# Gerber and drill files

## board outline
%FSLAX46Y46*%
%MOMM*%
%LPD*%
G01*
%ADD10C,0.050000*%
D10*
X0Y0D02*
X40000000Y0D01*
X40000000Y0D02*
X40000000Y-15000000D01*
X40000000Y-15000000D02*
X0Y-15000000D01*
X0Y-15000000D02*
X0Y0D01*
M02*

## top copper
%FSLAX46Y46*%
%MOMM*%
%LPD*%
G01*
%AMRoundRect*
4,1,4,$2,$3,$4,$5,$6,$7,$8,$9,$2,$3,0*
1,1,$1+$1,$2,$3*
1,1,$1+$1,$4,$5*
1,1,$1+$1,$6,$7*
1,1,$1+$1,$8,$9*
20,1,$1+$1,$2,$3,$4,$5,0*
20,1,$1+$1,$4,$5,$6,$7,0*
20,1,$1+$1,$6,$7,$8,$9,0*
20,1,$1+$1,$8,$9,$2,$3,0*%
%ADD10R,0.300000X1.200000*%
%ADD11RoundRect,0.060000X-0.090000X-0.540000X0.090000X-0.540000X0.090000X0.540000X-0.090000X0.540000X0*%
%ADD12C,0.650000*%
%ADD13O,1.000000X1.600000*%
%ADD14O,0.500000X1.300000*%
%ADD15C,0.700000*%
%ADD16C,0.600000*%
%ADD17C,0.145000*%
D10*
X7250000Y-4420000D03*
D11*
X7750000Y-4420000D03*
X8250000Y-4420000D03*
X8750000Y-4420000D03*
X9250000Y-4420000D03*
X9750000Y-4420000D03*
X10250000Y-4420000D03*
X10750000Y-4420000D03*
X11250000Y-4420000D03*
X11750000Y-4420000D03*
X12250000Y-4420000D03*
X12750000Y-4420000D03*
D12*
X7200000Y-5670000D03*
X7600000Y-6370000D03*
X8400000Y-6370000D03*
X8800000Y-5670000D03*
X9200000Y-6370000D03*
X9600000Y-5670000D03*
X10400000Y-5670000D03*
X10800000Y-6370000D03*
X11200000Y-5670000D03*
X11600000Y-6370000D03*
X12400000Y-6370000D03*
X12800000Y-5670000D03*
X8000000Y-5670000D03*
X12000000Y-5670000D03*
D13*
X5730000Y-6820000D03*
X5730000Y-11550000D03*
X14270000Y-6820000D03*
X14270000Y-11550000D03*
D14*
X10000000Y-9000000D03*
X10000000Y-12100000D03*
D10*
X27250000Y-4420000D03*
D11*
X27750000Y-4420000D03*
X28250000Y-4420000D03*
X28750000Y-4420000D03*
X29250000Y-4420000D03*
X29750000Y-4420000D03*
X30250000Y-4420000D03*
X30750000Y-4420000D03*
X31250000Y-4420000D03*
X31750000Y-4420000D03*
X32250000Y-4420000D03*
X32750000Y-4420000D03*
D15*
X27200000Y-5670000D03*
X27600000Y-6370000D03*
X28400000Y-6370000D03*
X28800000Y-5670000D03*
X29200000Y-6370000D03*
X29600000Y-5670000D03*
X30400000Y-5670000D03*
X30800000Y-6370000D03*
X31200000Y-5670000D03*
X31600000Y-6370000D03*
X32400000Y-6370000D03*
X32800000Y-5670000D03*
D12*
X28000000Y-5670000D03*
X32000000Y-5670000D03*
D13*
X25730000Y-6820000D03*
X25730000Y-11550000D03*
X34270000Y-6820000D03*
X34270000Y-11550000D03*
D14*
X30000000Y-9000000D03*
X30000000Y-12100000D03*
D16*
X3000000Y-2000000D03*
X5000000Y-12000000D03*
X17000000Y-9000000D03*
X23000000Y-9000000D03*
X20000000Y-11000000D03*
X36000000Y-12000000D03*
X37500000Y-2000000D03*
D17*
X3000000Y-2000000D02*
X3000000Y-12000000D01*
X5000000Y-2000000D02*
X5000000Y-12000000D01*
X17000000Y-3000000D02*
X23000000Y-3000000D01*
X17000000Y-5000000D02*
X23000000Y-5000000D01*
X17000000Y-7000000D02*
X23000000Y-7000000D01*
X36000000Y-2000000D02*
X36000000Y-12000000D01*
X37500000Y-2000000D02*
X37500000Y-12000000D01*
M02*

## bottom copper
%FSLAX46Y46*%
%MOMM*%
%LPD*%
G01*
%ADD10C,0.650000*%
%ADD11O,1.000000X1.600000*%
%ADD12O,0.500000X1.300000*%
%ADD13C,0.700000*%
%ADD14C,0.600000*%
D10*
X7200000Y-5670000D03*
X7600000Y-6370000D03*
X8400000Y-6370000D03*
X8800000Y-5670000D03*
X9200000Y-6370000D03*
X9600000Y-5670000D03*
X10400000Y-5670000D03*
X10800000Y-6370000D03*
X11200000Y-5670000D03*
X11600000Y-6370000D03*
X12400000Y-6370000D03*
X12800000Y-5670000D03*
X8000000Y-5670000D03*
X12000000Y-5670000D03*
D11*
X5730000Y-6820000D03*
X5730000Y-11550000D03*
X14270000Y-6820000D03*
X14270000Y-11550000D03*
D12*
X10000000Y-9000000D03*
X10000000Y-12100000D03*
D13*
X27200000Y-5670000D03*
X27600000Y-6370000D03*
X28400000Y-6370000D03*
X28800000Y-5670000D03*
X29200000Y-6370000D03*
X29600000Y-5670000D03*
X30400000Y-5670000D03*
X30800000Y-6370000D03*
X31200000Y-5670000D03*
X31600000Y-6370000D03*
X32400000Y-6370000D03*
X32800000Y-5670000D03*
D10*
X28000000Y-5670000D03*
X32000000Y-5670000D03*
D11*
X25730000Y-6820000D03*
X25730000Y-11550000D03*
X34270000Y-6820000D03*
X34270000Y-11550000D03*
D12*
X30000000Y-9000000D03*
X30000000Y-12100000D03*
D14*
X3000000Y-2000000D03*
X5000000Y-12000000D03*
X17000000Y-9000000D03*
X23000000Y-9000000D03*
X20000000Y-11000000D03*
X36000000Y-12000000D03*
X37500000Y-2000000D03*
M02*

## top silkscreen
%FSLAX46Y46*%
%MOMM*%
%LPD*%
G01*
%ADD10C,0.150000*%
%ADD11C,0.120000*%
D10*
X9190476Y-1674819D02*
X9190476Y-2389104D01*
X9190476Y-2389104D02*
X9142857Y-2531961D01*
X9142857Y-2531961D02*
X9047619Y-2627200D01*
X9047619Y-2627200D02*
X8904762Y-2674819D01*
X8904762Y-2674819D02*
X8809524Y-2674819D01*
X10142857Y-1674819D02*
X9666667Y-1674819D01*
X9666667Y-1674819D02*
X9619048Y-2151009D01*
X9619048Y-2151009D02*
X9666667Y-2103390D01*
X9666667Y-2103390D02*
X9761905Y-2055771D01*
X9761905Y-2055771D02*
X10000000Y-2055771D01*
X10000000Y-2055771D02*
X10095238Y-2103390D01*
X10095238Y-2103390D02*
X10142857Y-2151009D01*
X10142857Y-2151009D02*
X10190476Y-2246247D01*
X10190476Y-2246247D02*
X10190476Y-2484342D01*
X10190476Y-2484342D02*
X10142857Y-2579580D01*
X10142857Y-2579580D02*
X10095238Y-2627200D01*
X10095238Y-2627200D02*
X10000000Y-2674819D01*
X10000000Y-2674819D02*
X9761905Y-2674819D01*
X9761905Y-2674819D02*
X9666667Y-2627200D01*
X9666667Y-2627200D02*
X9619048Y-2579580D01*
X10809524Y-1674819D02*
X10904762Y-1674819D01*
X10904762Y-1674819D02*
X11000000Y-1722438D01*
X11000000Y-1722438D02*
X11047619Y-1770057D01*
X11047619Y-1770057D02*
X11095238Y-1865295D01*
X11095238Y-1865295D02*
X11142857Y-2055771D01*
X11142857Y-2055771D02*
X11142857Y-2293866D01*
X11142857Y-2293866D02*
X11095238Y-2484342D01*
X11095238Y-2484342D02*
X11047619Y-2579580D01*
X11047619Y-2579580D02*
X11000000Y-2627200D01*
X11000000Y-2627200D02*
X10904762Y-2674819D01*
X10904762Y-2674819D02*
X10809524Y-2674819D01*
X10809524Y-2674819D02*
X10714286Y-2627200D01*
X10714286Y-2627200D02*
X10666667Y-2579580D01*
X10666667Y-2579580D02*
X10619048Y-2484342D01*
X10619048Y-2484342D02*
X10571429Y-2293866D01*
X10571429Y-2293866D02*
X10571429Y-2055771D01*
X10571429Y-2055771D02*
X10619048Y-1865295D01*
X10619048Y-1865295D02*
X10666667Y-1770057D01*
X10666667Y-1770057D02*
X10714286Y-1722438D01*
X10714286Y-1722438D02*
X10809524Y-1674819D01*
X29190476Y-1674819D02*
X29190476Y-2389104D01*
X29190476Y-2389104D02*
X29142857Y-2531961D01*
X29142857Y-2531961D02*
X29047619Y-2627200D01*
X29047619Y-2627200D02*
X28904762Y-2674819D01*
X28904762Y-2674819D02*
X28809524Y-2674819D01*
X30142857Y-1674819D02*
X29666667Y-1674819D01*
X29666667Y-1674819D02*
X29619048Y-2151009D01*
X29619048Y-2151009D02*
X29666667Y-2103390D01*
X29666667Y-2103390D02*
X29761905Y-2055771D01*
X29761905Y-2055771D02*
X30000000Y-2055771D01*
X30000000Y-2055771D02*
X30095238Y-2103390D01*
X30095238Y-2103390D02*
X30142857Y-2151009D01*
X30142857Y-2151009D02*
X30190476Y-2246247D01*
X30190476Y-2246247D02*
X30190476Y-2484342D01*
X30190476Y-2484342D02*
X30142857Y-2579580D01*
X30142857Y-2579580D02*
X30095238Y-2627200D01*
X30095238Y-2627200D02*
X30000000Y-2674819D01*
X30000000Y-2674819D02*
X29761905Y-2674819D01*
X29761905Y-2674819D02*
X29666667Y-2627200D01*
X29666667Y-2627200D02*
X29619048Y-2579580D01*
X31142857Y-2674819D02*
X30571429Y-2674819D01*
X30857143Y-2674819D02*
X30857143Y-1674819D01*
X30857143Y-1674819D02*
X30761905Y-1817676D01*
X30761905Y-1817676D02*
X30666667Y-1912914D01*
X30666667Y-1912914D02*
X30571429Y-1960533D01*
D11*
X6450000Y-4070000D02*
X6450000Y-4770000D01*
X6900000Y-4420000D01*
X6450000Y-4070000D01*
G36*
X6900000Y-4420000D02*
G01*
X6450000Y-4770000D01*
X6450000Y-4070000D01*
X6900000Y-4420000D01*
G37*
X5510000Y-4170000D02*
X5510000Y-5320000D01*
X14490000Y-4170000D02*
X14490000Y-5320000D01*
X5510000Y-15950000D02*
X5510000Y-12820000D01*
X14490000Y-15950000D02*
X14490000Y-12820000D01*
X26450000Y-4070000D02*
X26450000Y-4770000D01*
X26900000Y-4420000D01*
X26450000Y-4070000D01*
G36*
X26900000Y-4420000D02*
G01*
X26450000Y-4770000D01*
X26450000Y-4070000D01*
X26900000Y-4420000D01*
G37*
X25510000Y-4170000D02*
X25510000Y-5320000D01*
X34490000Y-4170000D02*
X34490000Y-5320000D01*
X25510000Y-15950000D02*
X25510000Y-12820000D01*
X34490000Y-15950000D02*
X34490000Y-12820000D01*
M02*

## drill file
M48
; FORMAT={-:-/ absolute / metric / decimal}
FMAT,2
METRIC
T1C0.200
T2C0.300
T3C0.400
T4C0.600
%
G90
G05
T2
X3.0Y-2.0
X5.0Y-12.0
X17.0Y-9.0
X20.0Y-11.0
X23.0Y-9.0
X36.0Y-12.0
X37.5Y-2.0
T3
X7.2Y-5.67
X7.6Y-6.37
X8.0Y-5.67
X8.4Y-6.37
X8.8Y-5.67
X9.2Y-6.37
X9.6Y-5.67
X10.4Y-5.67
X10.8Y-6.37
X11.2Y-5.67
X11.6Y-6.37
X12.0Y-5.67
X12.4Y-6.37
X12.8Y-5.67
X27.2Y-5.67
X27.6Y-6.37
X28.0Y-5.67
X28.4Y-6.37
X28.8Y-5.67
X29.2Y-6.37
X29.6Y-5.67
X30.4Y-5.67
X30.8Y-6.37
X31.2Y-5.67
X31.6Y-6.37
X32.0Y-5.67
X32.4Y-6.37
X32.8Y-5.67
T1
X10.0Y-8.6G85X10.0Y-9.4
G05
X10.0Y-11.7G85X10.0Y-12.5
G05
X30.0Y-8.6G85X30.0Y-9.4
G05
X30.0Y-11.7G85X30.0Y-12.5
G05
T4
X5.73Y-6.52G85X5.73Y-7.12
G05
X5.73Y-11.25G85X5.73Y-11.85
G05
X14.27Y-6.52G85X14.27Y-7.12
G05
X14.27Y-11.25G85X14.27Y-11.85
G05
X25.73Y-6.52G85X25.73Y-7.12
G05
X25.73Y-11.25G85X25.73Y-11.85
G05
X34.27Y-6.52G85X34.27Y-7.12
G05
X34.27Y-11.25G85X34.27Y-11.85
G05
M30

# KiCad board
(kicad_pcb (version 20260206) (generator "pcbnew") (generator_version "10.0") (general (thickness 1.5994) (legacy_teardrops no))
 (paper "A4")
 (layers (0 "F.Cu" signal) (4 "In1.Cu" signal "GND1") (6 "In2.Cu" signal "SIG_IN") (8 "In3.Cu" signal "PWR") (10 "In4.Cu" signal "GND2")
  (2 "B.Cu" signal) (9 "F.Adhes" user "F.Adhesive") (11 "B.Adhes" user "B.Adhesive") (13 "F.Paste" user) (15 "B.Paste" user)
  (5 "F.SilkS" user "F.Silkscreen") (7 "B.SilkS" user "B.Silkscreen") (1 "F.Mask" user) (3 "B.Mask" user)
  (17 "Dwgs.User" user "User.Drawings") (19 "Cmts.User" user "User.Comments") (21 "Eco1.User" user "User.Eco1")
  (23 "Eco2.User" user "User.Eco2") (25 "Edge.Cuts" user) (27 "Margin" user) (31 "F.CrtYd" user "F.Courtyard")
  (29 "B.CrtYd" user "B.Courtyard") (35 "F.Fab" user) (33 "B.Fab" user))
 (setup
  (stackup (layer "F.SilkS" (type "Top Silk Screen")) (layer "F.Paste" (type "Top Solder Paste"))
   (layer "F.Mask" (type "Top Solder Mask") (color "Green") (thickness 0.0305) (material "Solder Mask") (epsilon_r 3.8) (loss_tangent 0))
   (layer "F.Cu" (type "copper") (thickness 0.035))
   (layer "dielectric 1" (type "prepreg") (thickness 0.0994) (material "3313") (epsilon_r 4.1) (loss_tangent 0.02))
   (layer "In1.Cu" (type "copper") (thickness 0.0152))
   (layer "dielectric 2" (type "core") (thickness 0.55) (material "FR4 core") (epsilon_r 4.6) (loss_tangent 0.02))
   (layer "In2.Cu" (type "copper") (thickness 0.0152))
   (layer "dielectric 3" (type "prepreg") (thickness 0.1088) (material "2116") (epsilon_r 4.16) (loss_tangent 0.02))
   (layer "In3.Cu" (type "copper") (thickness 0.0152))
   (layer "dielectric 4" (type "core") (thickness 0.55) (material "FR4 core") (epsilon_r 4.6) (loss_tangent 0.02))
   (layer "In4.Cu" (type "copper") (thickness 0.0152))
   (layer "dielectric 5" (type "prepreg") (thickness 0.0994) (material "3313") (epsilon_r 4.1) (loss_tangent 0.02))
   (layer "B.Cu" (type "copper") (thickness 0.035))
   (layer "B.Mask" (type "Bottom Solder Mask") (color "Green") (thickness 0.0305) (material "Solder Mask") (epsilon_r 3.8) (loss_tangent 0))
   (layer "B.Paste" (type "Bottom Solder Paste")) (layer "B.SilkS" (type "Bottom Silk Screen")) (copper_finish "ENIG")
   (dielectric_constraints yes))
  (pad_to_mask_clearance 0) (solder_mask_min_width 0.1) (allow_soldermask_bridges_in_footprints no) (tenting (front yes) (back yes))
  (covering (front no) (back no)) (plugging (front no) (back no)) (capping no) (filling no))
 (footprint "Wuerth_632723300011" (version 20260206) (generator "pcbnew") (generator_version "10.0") (layer "F.Cu") (at 10 4.42)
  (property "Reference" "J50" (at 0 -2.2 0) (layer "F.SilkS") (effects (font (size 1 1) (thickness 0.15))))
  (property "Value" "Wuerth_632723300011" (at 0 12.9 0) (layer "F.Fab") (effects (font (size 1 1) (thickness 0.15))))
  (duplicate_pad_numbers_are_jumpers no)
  (fp_poly (pts (xy -3.55 -0.35) (xy -3.55 0.35) (xy -3.1 0)) (stroke (width 0.12) (type solid)) (fill yes) (layer "F.SilkS"))
  (fp_line (start -4.49 -0.25) (end -4.49 0.9) (stroke (width 0.12) (type solid)) (layer "F.SilkS"))
  (fp_line (start 4.49 -0.25) (end 4.49 0.9) (stroke (width 0.12) (type solid)) (layer "F.SilkS"))
  (fp_line (start -4.49 11.53) (end -4.49 8.4) (stroke (width 0.12) (type solid)) (layer "F.SilkS"))
  (fp_line (start 4.49 11.53) (end 4.49 8.4) (stroke (width 0.12) (type solid)) (layer "F.SilkS"))
  (pad "A1" smd rect (at -2.75 0) (size 0.3 1.2) (layers "F.Cu" "F.Mask" "F.Paste"))
  (pad "A2" smd roundrect (at -2.25 0) (size 0.3 1.2) (layers "F.Cu" "F.Mask" "F.Paste") (roundrect_rratio 0.2))
  (pad "A3" smd roundrect (at -1.75 0) (size 0.3 1.2) (layers "F.Cu" "F.Mask" "F.Paste") (roundrect_rratio 0.2))
  (pad "A4" smd roundrect (at -1.25 0) (size 0.3 1.2) (layers "F.Cu" "F.Mask" "F.Paste") (roundrect_rratio 0.2))
  (pad "A5" smd roundrect (at -0.75 0) (size 0.3 1.2) (layers "F.Cu" "F.Mask" "F.Paste") (roundrect_rratio 0.2))
  (pad "A6" smd roundrect (at -0.25 0) (size 0.3 1.2) (layers "F.Cu" "F.Mask" "F.Paste") (roundrect_rratio 0.2))
  (pad "A7" smd roundrect (at 0.25 0) (size 0.3 1.2) (layers "F.Cu" "F.Mask" "F.Paste") (roundrect_rratio 0.2))
  (pad "A8" smd roundrect (at 0.75 0) (size 0.3 1.2) (layers "F.Cu" "F.Mask" "F.Paste") (roundrect_rratio 0.2))
  (pad "A9" smd roundrect (at 1.25 0) (size 0.3 1.2) (layers "F.Cu" "F.Mask" "F.Paste") (roundrect_rratio 0.2))
  (pad "A10" smd roundrect (at 1.75 0) (size 0.3 1.2) (layers "F.Cu" "F.Mask" "F.Paste") (roundrect_rratio 0.2))
  (pad "A11" smd roundrect (at 2.25 0) (size 0.3 1.2) (layers "F.Cu" "F.Mask" "F.Paste") (roundrect_rratio 0.2))
  (pad "A12" smd roundrect (at 2.75 0) (size 0.3 1.2) (layers "F.Cu" "F.Mask" "F.Paste") (roundrect_rratio 0.2))
  (pad "B12" thru_hole circle (at -2.8 1.25) (size 0.65 0.65) (drill 0.4) (layers "*.Cu" "*.Mask") (remove_unused_layers no))
  (pad "B11" thru_hole circle (at -2.4 1.95) (size 0.65 0.65) (drill 0.4) (layers "*.Cu" "*.Mask") (remove_unused_layers no))
  (pad "B10" thru_hole circle (at -1.6 1.95) (size 0.65 0.65) (drill 0.4) (layers "*.Cu" "*.Mask") (remove_unused_layers no))
  (pad "B9" thru_hole circle (at -1.2 1.25) (size 0.65 0.65) (drill 0.4) (layers "*.Cu" "*.Mask") (remove_unused_layers no))
  (pad "B8" thru_hole circle (at -0.8 1.95) (size 0.65 0.65) (drill 0.4) (layers "*.Cu" "*.Mask") (remove_unused_layers no))
  (pad "B7" thru_hole circle (at -0.4 1.25) (size 0.65 0.65) (drill 0.4) (layers "*.Cu" "*.Mask") (remove_unused_layers no))
  (pad "B6" thru_hole circle (at 0.4 1.25) (size 0.65 0.65) (drill 0.4) (layers "*.Cu" "*.Mask") (remove_unused_layers no))
  (pad "B5" thru_hole circle (at 0.8 1.95) (size 0.65 0.65) (drill 0.4) (layers "*.Cu" "*.Mask") (remove_unused_layers no))
  (pad "B4" thru_hole circle (at 1.2 1.25) (size 0.65 0.65) (drill 0.4) (layers "*.Cu" "*.Mask") (remove_unused_layers no))
  (pad "B3" thru_hole circle (at 1.6 1.95) (size 0.65 0.65) (drill 0.4) (layers "*.Cu" "*.Mask") (remove_unused_layers no))
  (pad "B2" thru_hole circle (at 2.4 1.95) (size 0.65 0.65) (drill 0.4) (layers "*.Cu" "*.Mask") (remove_unused_layers no))
  (pad "B1" thru_hole circle (at 2.8 1.25) (size 0.65 0.65) (drill 0.4) (layers "*.Cu" "*.Mask") (remove_unused_layers no))
  (pad "S1" thru_hole circle (at -2.0 1.25) (size 0.65 0.65) (drill 0.4) (layers "*.Cu" "*.Mask") (remove_unused_layers no))
  (pad "S1" thru_hole circle (at 2.0 1.25) (size 0.65 0.65) (drill 0.4) (layers "*.Cu" "*.Mask") (remove_unused_layers no))
  (pad "S1" thru_hole oval (at -4.27 2.4) (size 1.0 1.6) (drill oval 0.6 1.2) (layers "*.Cu" "*.Mask") (remove_unused_layers no))
  (pad "S1" thru_hole oval (at -4.27 7.13) (size 1.0 1.6) (drill oval 0.6 1.2) (layers "*.Cu" "*.Mask") (remove_unused_layers no))
  (pad "S1" thru_hole oval (at 4.27 2.4) (size 1.0 1.6) (drill oval 0.6 1.2) (layers "*.Cu" "*.Mask") (remove_unused_layers no))
  (pad "S1" thru_hole oval (at 4.27 7.13) (size 1.0 1.6) (drill oval 0.6 1.2) (layers "*.Cu" "*.Mask") (remove_unused_layers no))
  (pad "S1" thru_hole oval (at 0 4.58) (size 0.5 1.3) (drill oval 0.2 1.0) (layers "*.Cu" "*.Mask") (remove_unused_layers no))
  (pad "S1" thru_hole oval (at 0 7.68) (size 0.5 1.3) (drill oval 0.2 1.0) (layers "*.Cu" "*.Mask") (remove_unused_layers no)))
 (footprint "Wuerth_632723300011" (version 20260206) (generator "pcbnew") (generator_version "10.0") (layer "F.Cu") (at 30 4.42)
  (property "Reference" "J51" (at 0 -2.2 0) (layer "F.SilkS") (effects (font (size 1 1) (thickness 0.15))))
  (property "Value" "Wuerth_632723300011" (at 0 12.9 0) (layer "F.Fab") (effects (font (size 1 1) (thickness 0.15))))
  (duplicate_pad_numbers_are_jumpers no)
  (fp_poly (pts (xy -3.55 -0.35) (xy -3.55 0.35) (xy -3.1 0)) (stroke (width 0.12) (type solid)) (fill yes) (layer "F.SilkS"))
  (fp_line (start -4.49 -0.25) (end -4.49 0.9) (stroke (width 0.12) (type solid)) (layer "F.SilkS"))
  (fp_line (start 4.49 -0.25) (end 4.49 0.9) (stroke (width 0.12) (type solid)) (layer "F.SilkS"))
  (fp_line (start -4.49 11.53) (end -4.49 8.4) (stroke (width 0.12) (type solid)) (layer "F.SilkS"))
  (fp_line (start 4.49 11.53) (end 4.49 8.4) (stroke (width 0.12) (type solid)) (layer "F.SilkS"))
  (pad "A1" smd rect (at -2.75 0) (size 0.3 1.2) (layers "F.Cu" "F.Mask" "F.Paste"))
  (pad "A2" smd roundrect (at -2.25 0) (size 0.3 1.2) (layers "F.Cu" "F.Mask" "F.Paste") (roundrect_rratio 0.2))
  (pad "A3" smd roundrect (at -1.75 0) (size 0.3 1.2) (layers "F.Cu" "F.Mask" "F.Paste") (roundrect_rratio 0.2))
  (pad "A4" smd roundrect (at -1.25 0) (size 0.3 1.2) (layers "F.Cu" "F.Mask" "F.Paste") (roundrect_rratio 0.2))
  (pad "A5" smd roundrect (at -0.75 0) (size 0.3 1.2) (layers "F.Cu" "F.Mask" "F.Paste") (roundrect_rratio 0.2))
  (pad "A6" smd roundrect (at -0.25 0) (size 0.3 1.2) (layers "F.Cu" "F.Mask" "F.Paste") (roundrect_rratio 0.2))
  (pad "A7" smd roundrect (at 0.25 0) (size 0.3 1.2) (layers "F.Cu" "F.Mask" "F.Paste") (roundrect_rratio 0.2))
  (pad "A8" smd roundrect (at 0.75 0) (size 0.3 1.2) (layers "F.Cu" "F.Mask" "F.Paste") (roundrect_rratio 0.2))
  (pad "A9" smd roundrect (at 1.25 0) (size 0.3 1.2) (layers "F.Cu" "F.Mask" "F.Paste") (roundrect_rratio 0.2))
  (pad "A10" smd roundrect (at 1.75 0) (size 0.3 1.2) (layers "F.Cu" "F.Mask" "F.Paste") (roundrect_rratio 0.2))
  (pad "A11" smd roundrect (at 2.25 0) (size 0.3 1.2) (layers "F.Cu" "F.Mask" "F.Paste") (roundrect_rratio 0.2))
  (pad "A12" smd roundrect (at 2.75 0) (size 0.3 1.2) (layers "F.Cu" "F.Mask" "F.Paste") (roundrect_rratio 0.2))
  (pad "B12" thru_hole circle (at -2.8 1.25) (size 0.7 0.7) (drill 0.4) (layers "*.Cu" "*.Mask") (remove_unused_layers no))
  (pad "B11" thru_hole circle (at -2.4 1.95) (size 0.7 0.7) (drill 0.4) (layers "*.Cu" "*.Mask") (remove_unused_layers no))
  (pad "B10" thru_hole circle (at -1.6 1.95) (size 0.7 0.7) (drill 0.4) (layers "*.Cu" "*.Mask") (remove_unused_layers no))
  (pad "B9" thru_hole circle (at -1.2 1.25) (size 0.7 0.7) (drill 0.4) (layers "*.Cu" "*.Mask") (remove_unused_layers no))
  (pad "B8" thru_hole circle (at -0.8 1.95) (size 0.7 0.7) (drill 0.4) (layers "*.Cu" "*.Mask") (remove_unused_layers no))
  (pad "B7" thru_hole circle (at -0.4 1.25) (size 0.7 0.7) (drill 0.4) (layers "*.Cu" "*.Mask") (remove_unused_layers no))
  (pad "B6" thru_hole circle (at 0.4 1.25) (size 0.7 0.7) (drill 0.4) (layers "*.Cu" "*.Mask") (remove_unused_layers no))
  (pad "B5" thru_hole circle (at 0.8 1.95) (size 0.7 0.7) (drill 0.4) (layers "*.Cu" "*.Mask") (remove_unused_layers no))
  (pad "B4" thru_hole circle (at 1.2 1.25) (size 0.7 0.7) (drill 0.4) (layers "*.Cu" "*.Mask") (remove_unused_layers no))
  (pad "B3" thru_hole circle (at 1.6 1.95) (size 0.7 0.7) (drill 0.4) (layers "*.Cu" "*.Mask") (remove_unused_layers no))
  (pad "B2" thru_hole circle (at 2.4 1.95) (size 0.7 0.7) (drill 0.4) (layers "*.Cu" "*.Mask") (remove_unused_layers no))
  (pad "B1" thru_hole circle (at 2.8 1.25) (size 0.7 0.7) (drill 0.4) (layers "*.Cu" "*.Mask") (remove_unused_layers no))
  (pad "S1" thru_hole circle (at -2.0 1.25) (size 0.65 0.65) (drill 0.4) (layers "*.Cu" "*.Mask") (remove_unused_layers no))
  (pad "S1" thru_hole circle (at 2.0 1.25) (size 0.65 0.65) (drill 0.4) (layers "*.Cu" "*.Mask") (remove_unused_layers no))
  (pad "S1" thru_hole oval (at -4.27 2.4) (size 1.0 1.6) (drill oval 0.6 1.2) (layers "*.Cu" "*.Mask") (remove_unused_layers no))
  (pad "S1" thru_hole oval (at -4.27 7.13) (size 1.0 1.6) (drill oval 0.6 1.2) (layers "*.Cu" "*.Mask") (remove_unused_layers no))
  (pad "S1" thru_hole oval (at 4.27 2.4) (size 1.0 1.6) (drill oval 0.6 1.2) (layers "*.Cu" "*.Mask") (remove_unused_layers no))
  (pad "S1" thru_hole oval (at 4.27 7.13) (size 1.0 1.6) (drill oval 0.6 1.2) (layers "*.Cu" "*.Mask") (remove_unused_layers no))
  (pad "S1" thru_hole oval (at 0 4.58) (size 0.5 1.3) (drill oval 0.2 1.0) (layers "*.Cu" "*.Mask") (remove_unused_layers no))
  (pad "S1" thru_hole oval (at 0 7.68) (size 0.5 1.3) (drill oval 0.2 1.0) (layers "*.Cu" "*.Mask") (remove_unused_layers no)))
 (gr_line (start 0 0) (end 40 0) (stroke (width 0.05) (type default)) (layer "Edge.Cuts"))
 (gr_line (start 40 0) (end 40 15) (stroke (width 0.05) (type default)) (layer "Edge.Cuts"))
 (gr_line (start 40 15) (end 0 15) (stroke (width 0.05) (type default)) (layer "Edge.Cuts"))
 (gr_line (start 0 15) (end 0 0) (stroke (width 0.05) (type default)) (layer "Edge.Cuts"))
 (segment (start 3 2) (end 3 12) (width 0.145) (layer "F.Cu"))
 (segment (start 5 2) (end 5 12) (width 0.145) (layer "F.Cu"))
 (segment (start 17 3) (end 23 3) (width 0.145) (layer "F.Cu"))
 (segment (start 17 5) (end 23 5) (width 0.145) (layer "F.Cu"))
 (segment (start 17 7) (end 23 7) (width 0.145) (layer "F.Cu"))
 (segment (start 36 2) (end 36 12) (width 0.145) (layer "F.Cu"))
 (segment (start 37.5 2) (end 37.5 12) (width 0.145) (layer "F.Cu")) (via (at 3 2) (size 0.6) (drill 0.3) (layers "F.Cu" "B.Cu"))
 (via (at 5 12) (size 0.6) (drill 0.3) (layers "F.Cu" "B.Cu"))
 (via (at 17 9) (size 0.6) (drill 0.3) (layers "F.Cu" "B.Cu"))
 (via (at 23 9) (size 0.6) (drill 0.3) (layers "F.Cu" "B.Cu"))
 (via (at 20 11) (size 0.6) (drill 0.3) (layers "F.Cu" "B.Cu"))
 (via (at 36 12) (size 0.6) (drill 0.3) (layers "F.Cu" "B.Cu"))
 (via (at 37.5 2) (size 0.6) (drill 0.3) (layers "F.Cu" "B.Cu")))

